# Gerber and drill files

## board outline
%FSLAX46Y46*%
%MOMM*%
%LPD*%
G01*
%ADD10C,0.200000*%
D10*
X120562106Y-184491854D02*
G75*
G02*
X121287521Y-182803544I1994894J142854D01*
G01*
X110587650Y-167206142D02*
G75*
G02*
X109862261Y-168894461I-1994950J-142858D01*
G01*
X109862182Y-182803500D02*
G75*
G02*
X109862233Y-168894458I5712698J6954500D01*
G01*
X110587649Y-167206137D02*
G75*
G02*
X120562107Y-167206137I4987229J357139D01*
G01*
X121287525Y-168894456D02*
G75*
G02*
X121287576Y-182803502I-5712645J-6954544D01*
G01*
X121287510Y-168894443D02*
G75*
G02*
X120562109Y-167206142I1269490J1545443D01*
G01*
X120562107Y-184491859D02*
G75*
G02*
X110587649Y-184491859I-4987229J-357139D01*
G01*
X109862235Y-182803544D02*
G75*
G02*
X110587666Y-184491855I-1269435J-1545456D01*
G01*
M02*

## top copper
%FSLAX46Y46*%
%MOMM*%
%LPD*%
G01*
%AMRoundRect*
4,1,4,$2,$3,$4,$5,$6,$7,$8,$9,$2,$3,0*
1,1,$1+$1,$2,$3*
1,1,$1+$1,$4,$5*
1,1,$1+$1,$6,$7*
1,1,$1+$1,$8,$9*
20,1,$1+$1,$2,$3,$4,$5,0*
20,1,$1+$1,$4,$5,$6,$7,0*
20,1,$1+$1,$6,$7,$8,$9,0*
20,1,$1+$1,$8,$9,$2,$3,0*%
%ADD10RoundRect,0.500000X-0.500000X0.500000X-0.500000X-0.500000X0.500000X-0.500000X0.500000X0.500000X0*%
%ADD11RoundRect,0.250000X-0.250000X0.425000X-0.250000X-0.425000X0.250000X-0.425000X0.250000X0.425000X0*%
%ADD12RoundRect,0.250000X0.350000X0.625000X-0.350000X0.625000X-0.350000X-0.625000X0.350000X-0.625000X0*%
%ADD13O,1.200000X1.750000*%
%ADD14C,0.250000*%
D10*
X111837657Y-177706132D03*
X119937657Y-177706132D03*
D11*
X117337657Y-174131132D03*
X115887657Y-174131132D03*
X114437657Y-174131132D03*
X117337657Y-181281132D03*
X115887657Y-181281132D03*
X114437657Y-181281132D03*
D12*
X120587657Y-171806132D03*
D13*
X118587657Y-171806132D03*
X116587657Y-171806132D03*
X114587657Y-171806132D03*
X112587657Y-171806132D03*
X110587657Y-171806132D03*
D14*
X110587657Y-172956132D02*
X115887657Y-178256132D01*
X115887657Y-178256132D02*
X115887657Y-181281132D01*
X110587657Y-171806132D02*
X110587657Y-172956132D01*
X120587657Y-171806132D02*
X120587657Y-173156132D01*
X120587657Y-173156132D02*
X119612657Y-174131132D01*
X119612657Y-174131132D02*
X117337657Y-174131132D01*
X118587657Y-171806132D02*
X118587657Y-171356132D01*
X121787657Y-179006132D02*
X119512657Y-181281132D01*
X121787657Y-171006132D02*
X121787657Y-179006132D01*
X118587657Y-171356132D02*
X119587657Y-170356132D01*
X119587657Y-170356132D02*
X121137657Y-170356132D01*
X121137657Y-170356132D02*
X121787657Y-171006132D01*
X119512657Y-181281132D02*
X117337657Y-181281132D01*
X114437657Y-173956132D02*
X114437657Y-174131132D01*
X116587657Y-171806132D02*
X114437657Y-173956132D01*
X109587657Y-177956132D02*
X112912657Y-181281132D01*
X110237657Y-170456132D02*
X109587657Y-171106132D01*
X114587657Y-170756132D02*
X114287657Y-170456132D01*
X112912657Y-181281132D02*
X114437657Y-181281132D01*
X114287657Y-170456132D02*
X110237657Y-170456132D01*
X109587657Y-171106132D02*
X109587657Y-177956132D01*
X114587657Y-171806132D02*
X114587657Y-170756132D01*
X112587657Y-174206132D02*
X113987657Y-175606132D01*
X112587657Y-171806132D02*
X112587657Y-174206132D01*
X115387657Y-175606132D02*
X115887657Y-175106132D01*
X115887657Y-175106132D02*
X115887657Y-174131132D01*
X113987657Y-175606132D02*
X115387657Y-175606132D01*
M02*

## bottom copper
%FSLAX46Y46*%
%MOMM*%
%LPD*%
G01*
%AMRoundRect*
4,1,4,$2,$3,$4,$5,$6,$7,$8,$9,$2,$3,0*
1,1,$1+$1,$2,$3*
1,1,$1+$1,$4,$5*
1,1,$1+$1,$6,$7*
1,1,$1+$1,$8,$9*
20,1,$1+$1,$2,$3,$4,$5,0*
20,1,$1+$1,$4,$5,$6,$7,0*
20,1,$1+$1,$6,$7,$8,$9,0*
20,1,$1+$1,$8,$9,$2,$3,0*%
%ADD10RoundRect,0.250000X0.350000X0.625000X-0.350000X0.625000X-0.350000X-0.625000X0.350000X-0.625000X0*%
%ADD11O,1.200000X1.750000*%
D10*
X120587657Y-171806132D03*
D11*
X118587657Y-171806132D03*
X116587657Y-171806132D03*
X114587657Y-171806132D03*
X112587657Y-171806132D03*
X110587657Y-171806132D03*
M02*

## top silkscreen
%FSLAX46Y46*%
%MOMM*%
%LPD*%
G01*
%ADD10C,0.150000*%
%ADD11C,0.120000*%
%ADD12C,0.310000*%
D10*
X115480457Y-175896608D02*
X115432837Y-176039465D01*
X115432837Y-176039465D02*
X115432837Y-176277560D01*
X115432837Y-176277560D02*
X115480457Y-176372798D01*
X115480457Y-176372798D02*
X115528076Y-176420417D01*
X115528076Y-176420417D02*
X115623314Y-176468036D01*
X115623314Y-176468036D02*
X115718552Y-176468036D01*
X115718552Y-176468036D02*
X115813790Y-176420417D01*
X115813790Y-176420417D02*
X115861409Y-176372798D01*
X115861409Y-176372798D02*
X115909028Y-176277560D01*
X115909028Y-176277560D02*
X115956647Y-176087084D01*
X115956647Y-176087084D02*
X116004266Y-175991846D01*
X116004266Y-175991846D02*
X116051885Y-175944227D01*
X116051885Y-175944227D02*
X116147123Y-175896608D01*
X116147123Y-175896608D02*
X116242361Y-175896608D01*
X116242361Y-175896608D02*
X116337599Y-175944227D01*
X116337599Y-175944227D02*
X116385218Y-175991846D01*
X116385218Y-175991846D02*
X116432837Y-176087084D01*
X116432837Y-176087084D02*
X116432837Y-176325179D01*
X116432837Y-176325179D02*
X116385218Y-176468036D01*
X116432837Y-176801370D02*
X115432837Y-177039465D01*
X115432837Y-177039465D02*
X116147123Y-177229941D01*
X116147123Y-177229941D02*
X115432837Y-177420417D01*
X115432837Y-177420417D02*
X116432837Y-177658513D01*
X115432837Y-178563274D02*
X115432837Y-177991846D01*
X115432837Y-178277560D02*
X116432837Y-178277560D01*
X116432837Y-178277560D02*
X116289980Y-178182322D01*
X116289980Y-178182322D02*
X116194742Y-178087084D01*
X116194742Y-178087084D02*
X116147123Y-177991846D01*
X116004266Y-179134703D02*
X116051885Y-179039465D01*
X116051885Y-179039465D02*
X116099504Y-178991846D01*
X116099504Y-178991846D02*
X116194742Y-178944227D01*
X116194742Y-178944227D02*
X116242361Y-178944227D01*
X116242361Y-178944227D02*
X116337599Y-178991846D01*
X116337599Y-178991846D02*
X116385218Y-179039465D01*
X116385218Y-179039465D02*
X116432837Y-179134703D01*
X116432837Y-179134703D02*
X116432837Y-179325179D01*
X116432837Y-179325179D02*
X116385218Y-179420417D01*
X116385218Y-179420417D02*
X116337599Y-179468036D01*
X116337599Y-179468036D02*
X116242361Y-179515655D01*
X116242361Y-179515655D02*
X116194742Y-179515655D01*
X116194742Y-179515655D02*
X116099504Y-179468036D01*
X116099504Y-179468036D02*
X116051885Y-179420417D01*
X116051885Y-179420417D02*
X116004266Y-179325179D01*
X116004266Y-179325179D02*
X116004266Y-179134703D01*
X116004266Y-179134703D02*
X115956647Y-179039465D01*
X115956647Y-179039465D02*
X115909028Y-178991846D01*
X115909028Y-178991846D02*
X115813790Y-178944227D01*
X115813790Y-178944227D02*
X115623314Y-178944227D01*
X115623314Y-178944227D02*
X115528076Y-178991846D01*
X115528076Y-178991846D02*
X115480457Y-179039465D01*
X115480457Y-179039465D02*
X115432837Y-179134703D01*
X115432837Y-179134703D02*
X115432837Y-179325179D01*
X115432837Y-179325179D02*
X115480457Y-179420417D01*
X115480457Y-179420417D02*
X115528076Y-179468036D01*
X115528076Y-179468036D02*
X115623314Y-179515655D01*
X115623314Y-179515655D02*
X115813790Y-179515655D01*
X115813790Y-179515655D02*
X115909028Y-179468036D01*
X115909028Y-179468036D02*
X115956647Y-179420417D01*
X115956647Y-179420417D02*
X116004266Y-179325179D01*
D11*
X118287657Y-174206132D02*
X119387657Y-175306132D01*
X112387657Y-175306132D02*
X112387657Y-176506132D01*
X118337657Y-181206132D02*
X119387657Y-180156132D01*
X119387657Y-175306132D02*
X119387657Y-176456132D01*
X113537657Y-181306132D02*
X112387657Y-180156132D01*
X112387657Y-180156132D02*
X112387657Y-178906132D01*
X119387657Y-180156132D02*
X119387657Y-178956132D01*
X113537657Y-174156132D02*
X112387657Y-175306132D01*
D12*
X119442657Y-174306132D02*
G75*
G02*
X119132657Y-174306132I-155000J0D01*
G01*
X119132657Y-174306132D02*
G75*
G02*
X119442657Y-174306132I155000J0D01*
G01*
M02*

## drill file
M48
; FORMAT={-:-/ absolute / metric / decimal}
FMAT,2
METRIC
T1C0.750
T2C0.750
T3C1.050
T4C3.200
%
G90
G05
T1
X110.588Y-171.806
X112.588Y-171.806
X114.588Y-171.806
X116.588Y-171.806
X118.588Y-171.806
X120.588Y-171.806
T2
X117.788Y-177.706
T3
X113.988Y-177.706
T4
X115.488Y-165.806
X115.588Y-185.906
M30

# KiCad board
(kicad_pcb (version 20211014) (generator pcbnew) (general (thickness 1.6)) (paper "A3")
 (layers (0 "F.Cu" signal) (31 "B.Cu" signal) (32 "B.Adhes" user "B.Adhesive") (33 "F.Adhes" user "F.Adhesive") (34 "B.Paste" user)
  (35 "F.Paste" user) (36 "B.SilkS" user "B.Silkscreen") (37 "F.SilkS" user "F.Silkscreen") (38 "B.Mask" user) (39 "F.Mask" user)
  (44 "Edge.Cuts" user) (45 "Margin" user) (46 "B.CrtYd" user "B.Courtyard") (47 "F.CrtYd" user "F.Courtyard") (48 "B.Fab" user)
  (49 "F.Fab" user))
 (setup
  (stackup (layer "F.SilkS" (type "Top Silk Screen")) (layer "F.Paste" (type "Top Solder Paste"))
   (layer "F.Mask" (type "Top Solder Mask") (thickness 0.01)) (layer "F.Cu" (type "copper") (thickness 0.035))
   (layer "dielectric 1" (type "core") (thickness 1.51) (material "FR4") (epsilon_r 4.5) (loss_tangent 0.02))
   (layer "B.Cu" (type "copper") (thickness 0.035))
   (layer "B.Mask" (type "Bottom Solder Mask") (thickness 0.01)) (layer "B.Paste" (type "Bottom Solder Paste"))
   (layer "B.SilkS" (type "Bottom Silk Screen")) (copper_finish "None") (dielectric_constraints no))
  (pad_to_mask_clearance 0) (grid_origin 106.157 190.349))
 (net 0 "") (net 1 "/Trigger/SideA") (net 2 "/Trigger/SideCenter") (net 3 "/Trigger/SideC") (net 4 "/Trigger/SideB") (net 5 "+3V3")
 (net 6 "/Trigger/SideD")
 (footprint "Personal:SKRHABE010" (layer "F.Cu") (at 115.887657 177.706132 -90)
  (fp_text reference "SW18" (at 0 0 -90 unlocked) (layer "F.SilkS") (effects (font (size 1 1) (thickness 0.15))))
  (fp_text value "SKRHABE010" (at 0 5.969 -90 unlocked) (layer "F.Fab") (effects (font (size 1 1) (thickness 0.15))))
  (fp_line (start -3.5 -2.4) (end -2.4 -3.5) (layer "F.SilkS") (width 0.12))
  (fp_line (start -2.4 3.5) (end -1.2 3.5) (layer "F.SilkS") (width 0.12))
  (fp_line (start 3.5 -2.45) (end 2.45 -3.5) (layer "F.SilkS") (width 0.12))
  (fp_line (start -2.4 -3.5) (end -1.25 -3.5) (layer "F.SilkS") (width 0.12))
  (fp_line (start 3.6 2.35) (end 2.45 3.5) (layer "F.SilkS") (width 0.12))
  (fp_line (start 2.45 3.5) (end 1.2 3.5) (layer "F.SilkS") (width 0.12))
  (fp_line (start 2.45 -3.5) (end 1.25 -3.5) (layer "F.SilkS") (width 0.12))
  (fp_line (start -3.55 2.35) (end -2.4 3.5) (layer "F.SilkS") (width 0.12))
  (fp_circle (center -3.4 -3.4) (end -3.15 -3.4) (layer "F.SilkS") (width 0.12) (fill solid))
  (pad "" np_thru_hole circle (at 0 1.9 270) (size 1 1) (drill 1.05) (layers F&B.Cu *.Mask))
  (pad "" smd roundrect (at 0 4.05 270) (size 2 2) (layers "F.Cu" "F.Paste" "F.Mask") (roundrect_rratio 0.25))
  (pad "" np_thru_hole circle (at 0 -1.9 270) (size 0.75 0.75) (drill 0.75) (layers F&B.Cu *.Mask))
  (pad "" smd roundrect (at 0 -4.05 270) (size 2 2) (layers "F.Cu" "F.Paste" "F.Mask") (roundrect_rratio 0.25))
  (pad "1" smd roundrect (at -3.575 -1.45 270) (size 1.35 1) (layers "F.Cu" "F.Paste" "F.Mask") (roundrect_rratio 0.25)
   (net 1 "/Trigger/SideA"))
  (pad "2" smd roundrect (at -3.575 0 270) (size 1.35 1) (layers "F.Cu" "F.Paste" "F.Mask") (roundrect_rratio 0.25)
   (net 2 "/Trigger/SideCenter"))
  (pad "3" smd roundrect (at -3.575 1.45 270) (size 1.35 1) (layers "F.Cu" "F.Paste" "F.Mask") (roundrect_rratio 0.25)
   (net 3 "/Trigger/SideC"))
  (pad "4" smd roundrect (at 3.575 -1.45 270) (size 1.35 1) (layers "F.Cu" "F.Paste" "F.Mask") (roundrect_rratio 0.25)
   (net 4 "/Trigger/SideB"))
  (pad "5" smd roundrect (at 3.575 0 270) (size 1.35 1) (layers "F.Cu" "F.Paste" "F.Mask") (roundrect_rratio 0.25) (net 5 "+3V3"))
  (pad "6" smd roundrect (at 3.575 1.45 270) (size 1.35 1) (layers "F.Cu" "F.Paste" "F.Mask") (roundrect_rratio 0.25)
   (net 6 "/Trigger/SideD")))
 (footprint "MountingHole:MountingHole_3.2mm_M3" (layer "F.Cu") (at 115.587657 185.906132)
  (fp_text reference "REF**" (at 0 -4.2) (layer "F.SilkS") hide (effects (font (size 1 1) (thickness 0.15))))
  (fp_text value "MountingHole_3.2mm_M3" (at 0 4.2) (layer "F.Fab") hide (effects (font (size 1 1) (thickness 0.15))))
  (pad "" np_thru_hole circle (at 0 0) (size 3.2 3.2) (drill 3.2) (layers *.Cu *.Mask)))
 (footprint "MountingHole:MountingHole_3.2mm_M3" (layer "F.Cu") (at 115.487657 165.806132)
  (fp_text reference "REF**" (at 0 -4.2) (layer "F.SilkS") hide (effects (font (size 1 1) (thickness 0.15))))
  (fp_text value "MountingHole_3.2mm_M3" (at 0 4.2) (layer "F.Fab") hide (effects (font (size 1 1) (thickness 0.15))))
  (pad "" np_thru_hole circle (at 0 0) (size 3.2 3.2) (drill 3.2) (layers *.Cu *.Mask)))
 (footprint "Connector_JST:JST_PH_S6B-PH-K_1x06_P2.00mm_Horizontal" (layer "B.Cu") (at 120.587657 171.806132 180)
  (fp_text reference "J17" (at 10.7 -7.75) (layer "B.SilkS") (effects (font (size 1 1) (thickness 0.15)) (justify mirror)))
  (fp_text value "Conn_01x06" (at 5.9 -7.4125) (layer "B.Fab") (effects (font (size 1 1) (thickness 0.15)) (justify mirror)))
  (pad "1" thru_hole roundrect (at 0 0 180) (size 1.2 1.75) (drill 0.75) (layers *.Cu *.Mask) (roundrect_rratio 0.208333)
   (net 1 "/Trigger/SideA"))
  (pad "2" thru_hole oval (at 2 0 180) (size 1.2 1.75) (drill 0.75) (layers *.Cu *.Mask) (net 4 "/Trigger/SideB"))
  (pad "3" thru_hole oval (at 4 0 180) (size 1.2 1.75) (drill 0.75) (layers *.Cu *.Mask) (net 3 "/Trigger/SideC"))
  (pad "4" thru_hole oval (at 6 0 180) (size 1.2 1.75) (drill 0.75) (layers *.Cu *.Mask) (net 6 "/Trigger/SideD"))
  (pad "5" thru_hole oval (at 8 0 180) (size 1.2 1.75) (drill 0.75) (layers *.Cu *.Mask) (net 2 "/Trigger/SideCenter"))
  (pad "6" thru_hole oval (at 10 0 180) (size 1.2 1.75) (drill 0.75) (layers *.Cu *.Mask) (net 5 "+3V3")))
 (gr_arc (start 120.562106 184.491854) (mid 120.719439 183.559456) (end 121.287521 182.803544) (layer "Edge.Cuts") (width 0.2))
 (gr_arc (start 110.58765 167.206142) (mid 110.430319 168.138533) (end 109.862246 168.894443) (layer "Edge.Cuts") (width 0.2))
 (gr_arc (start 109.862182 182.8035) (mid 106.574878 175.848966) (end 109.862231 168.894456) (layer "Edge.Cuts") (width 0.2))
 (gr_arc (start 110.587649 167.206137) (mid 115.574878 161.848998) (end 120.562107 167.206137) (layer "Edge.Cuts") (width 0.2))
 (gr_arc (start 121.287525 168.894456) (mid 124.574878 175.848966) (end 121.287574 182.8035) (layer "Edge.Cuts") (width 0.2))
 (gr_arc (start 121.28751 168.894443) (mid 120.719431 168.138536) (end 120.562106 167.206142) (layer "Edge.Cuts") (width 0.2))
 (gr_arc (start 120.562107 184.491859) (mid 115.574878 189.848998) (end 110.587649 184.491859) (layer "Edge.Cuts") (width 0.2))
 (gr_arc (start 109.862235 182.803544) (mid 110.430317 183.559456) (end 110.58765 184.491854) (layer "Edge.Cuts") (width 0.2))
 (segment (start 110.587657 172.956132) (end 115.887657 178.256132) (width 0.25) (layer "F.Cu") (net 5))
 (segment (start 115.887657 178.256132) (end 115.887657 181.281132) (width 0.25) (layer "F.Cu") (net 5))
 (segment (start 110.587657 171.806132) (end 110.587657 172.956132) (width 0.25) (layer "F.Cu") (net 5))
 (segment (start 120.587657 171.806132) (end 120.587657 173.156132) (width 0.25) (layer "F.Cu") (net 1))
 (segment (start 120.587657 173.156132) (end 119.612657 174.131132) (width 0.25) (layer "F.Cu") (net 1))
 (segment (start 119.612657 174.131132) (end 117.337657 174.131132) (width 0.25) (layer "F.Cu") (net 1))
 (segment (start 118.587657 171.806132) (end 118.587657 171.356132) (width 0.25) (layer "F.Cu") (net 4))
 (segment (start 121.787657 179.006132) (end 119.512657 181.281132) (width 0.25) (layer "F.Cu") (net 4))
 (segment (start 121.787657 171.006132) (end 121.787657 179.006132) (width 0.25) (layer "F.Cu") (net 4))
 (segment (start 118.587657 171.356132) (end 119.587657 170.356132) (width 0.25) (layer "F.Cu") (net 4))
 (segment (start 119.587657 170.356132) (end 121.137657 170.356132) (width 0.25) (layer "F.Cu") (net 4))
 (segment (start 121.137657 170.356132) (end 121.787657 171.006132) (width 0.25) (layer "F.Cu") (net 4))
 (segment (start 119.512657 181.281132) (end 117.337657 181.281132) (width 0.25) (layer "F.Cu") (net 4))
 (segment (start 114.437657 173.956132) (end 114.437657 174.131132) (width 0.25) (layer "F.Cu") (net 3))
 (segment (start 116.587657 171.806132) (end 114.437657 173.956132) (width 0.25) (layer "F.Cu") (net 3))
 (segment (start 109.587657 177.956132) (end 112.912657 181.281132) (width 0.25) (layer "F.Cu") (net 6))
 (segment (start 110.237657 170.456132) (end 109.587657 171.106132) (width 0.25) (layer "F.Cu") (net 6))
 (segment (start 114.587657 170.756132) (end 114.287657 170.456132) (width 0.25) (layer "F.Cu") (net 6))
 (segment (start 112.912657 181.281132) (end 114.437657 181.281132) (width 0.25) (layer "F.Cu") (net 6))
 (segment (start 114.287657 170.456132) (end 110.237657 170.456132) (width 0.25) (layer "F.Cu") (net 6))
 (segment (start 109.587657 171.106132) (end 109.587657 177.956132) (width 0.25) (layer "F.Cu") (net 6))
 (segment (start 114.587657 171.806132) (end 114.587657 170.756132) (width 0.25) (layer "F.Cu") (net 6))
 (segment (start 112.587657 174.206132) (end 113.987657 175.606132) (width 0.25) (layer "F.Cu") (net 2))
 (segment (start 112.587657 171.806132) (end 112.587657 174.206132) (width 0.25) (layer "F.Cu") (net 2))
 (segment (start 115.387657 175.606132) (end 115.887657 175.106132) (width 0.25) (layer "F.Cu") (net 2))
 (segment (start 115.887657 175.106132) (end 115.887657 174.131132) (width 0.25) (layer "F.Cu") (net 2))
 (segment (start 113.987657 175.606132) (end 115.387657 175.606132) (width 0.25) (layer "F.Cu") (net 2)))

